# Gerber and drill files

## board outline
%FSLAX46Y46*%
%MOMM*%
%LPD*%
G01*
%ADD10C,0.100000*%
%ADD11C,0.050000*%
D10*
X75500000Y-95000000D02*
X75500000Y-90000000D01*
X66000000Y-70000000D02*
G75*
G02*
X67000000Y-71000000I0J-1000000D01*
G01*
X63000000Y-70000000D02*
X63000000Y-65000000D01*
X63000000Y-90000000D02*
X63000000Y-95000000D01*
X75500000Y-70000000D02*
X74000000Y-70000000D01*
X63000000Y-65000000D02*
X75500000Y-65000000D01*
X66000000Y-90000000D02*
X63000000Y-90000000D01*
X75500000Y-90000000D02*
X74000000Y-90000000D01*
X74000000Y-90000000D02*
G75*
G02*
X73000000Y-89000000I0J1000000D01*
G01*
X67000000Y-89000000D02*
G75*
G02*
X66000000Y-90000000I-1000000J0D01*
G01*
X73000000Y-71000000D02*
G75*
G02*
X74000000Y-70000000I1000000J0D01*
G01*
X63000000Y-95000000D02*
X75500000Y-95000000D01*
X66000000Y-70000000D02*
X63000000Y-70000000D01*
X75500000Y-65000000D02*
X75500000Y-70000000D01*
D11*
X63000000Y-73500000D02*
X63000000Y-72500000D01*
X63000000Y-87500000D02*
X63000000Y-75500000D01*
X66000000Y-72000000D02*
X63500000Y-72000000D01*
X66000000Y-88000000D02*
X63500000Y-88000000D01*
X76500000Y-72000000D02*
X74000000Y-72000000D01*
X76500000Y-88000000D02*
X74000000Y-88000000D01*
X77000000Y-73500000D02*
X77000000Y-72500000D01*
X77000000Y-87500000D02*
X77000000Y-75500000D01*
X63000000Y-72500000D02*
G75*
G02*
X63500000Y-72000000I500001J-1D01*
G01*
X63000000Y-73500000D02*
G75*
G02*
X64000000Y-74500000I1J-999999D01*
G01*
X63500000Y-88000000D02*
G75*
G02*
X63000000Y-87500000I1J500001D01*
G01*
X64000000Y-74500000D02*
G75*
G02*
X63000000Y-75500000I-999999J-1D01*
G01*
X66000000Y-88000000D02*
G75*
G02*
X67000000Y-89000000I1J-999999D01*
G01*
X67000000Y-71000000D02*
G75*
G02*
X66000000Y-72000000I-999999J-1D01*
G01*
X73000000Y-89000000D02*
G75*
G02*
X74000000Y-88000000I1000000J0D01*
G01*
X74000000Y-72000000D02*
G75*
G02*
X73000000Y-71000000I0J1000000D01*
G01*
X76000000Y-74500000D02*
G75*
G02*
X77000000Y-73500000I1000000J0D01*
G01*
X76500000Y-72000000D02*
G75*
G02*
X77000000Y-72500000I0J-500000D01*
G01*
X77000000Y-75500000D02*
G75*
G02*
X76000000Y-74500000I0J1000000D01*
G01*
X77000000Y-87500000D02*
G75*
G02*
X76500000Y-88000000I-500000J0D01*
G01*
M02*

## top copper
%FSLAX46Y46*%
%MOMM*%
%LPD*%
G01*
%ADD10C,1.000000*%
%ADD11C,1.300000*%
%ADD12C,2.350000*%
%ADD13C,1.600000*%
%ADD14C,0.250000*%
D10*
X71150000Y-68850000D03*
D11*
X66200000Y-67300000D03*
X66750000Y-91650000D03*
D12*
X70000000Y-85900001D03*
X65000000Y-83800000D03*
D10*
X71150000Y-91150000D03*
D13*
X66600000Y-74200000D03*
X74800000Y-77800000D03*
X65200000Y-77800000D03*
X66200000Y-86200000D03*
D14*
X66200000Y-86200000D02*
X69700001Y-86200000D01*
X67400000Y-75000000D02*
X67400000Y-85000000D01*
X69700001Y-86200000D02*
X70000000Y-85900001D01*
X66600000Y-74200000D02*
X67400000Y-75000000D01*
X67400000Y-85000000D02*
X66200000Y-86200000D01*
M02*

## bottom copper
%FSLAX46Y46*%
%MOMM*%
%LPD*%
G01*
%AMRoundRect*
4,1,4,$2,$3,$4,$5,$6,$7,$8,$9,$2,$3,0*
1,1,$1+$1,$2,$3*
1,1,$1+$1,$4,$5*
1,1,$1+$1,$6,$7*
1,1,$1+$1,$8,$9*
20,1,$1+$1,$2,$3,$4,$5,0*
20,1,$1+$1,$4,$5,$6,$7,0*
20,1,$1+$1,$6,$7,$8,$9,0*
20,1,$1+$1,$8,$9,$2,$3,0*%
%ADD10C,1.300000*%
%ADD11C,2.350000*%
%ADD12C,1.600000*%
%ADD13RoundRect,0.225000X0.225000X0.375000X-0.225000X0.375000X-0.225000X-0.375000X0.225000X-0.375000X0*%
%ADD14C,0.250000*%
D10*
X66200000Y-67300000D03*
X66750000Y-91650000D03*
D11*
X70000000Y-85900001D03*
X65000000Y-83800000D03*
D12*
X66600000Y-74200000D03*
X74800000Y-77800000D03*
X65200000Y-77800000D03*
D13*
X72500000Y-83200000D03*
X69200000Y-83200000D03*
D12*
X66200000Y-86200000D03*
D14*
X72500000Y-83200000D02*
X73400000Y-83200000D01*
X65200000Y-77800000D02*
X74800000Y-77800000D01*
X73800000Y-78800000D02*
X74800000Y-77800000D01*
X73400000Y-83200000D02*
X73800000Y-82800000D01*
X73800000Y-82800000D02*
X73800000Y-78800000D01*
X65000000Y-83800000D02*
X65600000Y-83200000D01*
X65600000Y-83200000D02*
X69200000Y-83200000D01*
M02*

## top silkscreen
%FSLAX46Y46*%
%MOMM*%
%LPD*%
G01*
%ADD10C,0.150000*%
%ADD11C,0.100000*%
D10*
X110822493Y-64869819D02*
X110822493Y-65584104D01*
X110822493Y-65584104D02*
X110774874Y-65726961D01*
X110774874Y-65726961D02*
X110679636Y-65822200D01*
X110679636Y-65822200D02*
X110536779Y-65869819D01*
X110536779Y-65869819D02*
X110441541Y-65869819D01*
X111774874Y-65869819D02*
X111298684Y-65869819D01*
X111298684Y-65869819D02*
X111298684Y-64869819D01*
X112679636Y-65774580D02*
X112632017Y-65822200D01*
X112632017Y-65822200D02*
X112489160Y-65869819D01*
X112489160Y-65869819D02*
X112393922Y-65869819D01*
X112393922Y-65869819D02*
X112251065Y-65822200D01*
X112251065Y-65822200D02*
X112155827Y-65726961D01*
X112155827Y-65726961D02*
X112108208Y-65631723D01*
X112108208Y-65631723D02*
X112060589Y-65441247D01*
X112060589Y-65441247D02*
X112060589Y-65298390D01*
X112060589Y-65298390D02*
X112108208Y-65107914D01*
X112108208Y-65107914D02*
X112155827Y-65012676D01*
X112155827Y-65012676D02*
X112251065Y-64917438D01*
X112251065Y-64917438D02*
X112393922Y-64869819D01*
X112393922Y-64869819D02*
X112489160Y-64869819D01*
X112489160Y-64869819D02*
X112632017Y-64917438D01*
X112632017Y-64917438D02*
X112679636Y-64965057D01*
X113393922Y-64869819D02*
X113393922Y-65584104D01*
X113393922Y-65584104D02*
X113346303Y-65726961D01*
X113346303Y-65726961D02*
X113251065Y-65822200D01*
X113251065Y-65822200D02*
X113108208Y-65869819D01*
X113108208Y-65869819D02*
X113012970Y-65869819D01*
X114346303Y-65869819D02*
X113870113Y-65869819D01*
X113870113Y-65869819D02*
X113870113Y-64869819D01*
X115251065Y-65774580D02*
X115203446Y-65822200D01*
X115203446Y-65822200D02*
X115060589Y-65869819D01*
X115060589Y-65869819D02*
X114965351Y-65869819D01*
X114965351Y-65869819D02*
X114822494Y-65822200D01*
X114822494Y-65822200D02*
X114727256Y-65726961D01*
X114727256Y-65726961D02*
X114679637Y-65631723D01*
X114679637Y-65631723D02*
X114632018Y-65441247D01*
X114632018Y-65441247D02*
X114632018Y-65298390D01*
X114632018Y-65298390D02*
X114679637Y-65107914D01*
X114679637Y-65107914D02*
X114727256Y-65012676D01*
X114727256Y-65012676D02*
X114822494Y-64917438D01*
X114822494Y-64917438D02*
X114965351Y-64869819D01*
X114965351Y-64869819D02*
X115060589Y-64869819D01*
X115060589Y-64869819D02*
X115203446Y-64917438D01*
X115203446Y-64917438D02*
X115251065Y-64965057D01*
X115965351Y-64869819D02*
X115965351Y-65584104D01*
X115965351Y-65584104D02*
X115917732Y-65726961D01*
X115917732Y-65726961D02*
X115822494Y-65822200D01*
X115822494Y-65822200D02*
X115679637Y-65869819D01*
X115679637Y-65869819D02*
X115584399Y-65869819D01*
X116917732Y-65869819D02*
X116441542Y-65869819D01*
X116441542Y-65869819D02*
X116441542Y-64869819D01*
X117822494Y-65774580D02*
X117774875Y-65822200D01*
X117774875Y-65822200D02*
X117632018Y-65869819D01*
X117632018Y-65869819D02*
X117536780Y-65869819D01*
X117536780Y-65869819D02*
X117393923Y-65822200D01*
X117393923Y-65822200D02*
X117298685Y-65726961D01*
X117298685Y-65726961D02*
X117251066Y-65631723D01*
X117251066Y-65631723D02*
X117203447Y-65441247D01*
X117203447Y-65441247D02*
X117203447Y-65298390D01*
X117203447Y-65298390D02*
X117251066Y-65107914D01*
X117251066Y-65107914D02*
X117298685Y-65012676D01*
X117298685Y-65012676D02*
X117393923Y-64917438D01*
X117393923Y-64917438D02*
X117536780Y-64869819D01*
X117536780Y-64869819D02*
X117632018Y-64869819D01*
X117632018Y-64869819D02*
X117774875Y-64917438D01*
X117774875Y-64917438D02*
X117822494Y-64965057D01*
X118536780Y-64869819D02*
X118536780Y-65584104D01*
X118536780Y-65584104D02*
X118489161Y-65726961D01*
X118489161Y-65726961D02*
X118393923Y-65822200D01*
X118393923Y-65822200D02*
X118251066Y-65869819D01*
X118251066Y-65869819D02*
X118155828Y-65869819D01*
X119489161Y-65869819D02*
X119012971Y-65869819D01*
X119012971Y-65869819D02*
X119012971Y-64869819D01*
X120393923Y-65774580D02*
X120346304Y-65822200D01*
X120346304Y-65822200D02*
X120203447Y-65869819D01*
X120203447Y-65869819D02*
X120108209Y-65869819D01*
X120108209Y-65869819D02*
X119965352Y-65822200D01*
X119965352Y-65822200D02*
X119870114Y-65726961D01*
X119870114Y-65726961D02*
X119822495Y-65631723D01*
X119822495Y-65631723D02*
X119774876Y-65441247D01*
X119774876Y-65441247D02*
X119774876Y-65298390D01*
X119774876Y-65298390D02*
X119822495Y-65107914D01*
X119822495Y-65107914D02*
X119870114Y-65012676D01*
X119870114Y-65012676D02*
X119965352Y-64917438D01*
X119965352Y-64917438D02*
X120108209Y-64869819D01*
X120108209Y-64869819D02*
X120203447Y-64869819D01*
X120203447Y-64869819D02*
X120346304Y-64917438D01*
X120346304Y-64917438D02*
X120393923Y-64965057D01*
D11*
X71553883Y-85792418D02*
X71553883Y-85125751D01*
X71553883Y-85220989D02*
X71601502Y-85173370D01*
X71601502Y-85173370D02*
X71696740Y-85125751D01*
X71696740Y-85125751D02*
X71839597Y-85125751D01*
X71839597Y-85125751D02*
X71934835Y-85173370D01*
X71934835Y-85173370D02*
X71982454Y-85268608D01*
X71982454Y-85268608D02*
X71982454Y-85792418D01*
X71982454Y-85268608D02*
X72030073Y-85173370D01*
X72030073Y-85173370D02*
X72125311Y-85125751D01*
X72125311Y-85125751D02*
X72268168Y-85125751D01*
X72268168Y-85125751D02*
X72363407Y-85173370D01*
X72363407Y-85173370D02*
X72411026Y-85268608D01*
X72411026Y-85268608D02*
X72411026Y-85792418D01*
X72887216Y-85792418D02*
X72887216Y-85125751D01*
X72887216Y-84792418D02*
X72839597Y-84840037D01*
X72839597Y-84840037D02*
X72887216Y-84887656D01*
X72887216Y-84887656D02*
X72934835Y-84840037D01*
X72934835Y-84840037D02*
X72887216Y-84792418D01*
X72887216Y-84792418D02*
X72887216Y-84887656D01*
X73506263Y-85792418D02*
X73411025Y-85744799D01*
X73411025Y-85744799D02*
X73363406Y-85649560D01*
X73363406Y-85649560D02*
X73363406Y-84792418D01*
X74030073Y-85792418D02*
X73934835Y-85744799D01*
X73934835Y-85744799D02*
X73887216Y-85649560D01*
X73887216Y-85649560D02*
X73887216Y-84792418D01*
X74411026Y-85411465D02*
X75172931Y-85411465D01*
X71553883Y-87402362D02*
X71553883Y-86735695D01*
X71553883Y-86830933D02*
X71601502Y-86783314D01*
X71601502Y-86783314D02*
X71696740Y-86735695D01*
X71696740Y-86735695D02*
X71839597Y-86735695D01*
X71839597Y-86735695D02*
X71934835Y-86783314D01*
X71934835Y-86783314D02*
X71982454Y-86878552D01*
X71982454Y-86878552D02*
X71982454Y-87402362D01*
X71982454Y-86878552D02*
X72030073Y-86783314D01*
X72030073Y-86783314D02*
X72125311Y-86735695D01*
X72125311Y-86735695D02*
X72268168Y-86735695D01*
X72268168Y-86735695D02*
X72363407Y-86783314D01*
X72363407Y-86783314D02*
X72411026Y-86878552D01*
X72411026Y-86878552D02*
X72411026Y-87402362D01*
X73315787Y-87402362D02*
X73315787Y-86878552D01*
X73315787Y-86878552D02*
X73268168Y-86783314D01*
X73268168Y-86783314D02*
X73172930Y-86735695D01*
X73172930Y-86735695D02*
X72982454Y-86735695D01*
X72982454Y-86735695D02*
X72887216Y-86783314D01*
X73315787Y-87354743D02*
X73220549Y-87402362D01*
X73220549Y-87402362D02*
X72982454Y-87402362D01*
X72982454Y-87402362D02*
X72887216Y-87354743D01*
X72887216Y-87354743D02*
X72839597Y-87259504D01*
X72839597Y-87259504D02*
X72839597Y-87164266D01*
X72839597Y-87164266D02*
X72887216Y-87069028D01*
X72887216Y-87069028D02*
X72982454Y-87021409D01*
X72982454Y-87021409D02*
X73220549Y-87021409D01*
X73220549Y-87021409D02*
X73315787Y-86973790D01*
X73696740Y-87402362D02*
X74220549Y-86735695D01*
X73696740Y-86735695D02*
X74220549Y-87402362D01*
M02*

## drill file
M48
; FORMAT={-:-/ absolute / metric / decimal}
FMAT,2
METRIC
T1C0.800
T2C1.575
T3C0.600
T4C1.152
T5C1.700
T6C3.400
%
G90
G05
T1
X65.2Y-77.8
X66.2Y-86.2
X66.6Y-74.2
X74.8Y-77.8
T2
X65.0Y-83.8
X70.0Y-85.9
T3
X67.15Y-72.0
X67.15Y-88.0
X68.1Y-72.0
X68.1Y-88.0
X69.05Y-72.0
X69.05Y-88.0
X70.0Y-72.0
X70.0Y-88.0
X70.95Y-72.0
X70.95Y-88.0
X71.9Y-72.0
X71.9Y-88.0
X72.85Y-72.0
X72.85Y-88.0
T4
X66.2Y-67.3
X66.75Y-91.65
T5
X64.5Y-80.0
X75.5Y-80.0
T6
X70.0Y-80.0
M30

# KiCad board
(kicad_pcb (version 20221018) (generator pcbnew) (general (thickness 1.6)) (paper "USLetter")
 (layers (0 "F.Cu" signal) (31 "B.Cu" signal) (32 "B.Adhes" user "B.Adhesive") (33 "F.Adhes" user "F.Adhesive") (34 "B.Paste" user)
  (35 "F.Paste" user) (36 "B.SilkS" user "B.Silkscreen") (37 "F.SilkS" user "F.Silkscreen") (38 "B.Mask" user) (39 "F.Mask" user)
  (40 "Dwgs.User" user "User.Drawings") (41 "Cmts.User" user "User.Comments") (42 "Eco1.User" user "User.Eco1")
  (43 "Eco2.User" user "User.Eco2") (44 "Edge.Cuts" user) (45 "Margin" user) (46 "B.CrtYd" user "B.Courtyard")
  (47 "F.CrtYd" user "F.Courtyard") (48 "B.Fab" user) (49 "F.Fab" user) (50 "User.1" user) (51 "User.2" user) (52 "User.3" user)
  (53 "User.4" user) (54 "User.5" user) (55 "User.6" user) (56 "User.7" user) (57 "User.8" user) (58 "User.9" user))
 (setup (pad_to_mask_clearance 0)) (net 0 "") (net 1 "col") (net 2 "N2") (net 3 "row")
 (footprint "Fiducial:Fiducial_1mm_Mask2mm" (layer "F.Cu") (at 71.15 68.85 -90)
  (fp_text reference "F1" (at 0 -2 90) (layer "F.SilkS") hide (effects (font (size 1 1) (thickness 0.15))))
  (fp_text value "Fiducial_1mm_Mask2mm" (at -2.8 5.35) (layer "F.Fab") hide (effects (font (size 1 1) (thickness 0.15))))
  (pad "" smd circle (at 0 0 270) (size 1 1) (layers "F.Cu" "F.Mask") (solder_mask_margin 0.5) (clearance 0.5)))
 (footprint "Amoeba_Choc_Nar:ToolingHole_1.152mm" (layer "F.Cu") (at 66.2 67.3 -90) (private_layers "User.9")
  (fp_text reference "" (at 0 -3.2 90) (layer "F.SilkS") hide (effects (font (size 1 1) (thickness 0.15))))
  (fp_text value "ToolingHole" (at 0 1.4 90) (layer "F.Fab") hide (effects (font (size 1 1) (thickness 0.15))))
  (pad "" np_thru_hole circle (at 0 0 270) (size 1.3 1.3) (drill 1.152) (layers "F&B.Cu" "*.Mask") (solder_mask_margin 0.074)))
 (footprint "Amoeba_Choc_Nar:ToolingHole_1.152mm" (layer "F.Cu") (at 66.75 91.65 -90) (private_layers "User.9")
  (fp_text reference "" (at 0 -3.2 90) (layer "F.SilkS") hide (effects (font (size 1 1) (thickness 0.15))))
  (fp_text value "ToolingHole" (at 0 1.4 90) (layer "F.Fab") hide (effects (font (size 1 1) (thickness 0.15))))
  (pad "" np_thru_hole circle (at 0 0 270) (size 1.3 1.3) (drill 1.152) (layers "F&B.Cu" "*.Mask") (solder_mask_margin 0.074)))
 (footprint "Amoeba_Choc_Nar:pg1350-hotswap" (layer "F.Cu") (at 70 80) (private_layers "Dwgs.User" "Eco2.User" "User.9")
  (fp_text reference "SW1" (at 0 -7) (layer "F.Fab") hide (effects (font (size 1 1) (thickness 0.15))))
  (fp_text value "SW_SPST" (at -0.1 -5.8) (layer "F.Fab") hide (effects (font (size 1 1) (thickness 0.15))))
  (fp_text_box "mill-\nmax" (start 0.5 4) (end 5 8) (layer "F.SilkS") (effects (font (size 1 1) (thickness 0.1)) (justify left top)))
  (fp_line (start -7 -6.5) (end -7 -7.5) (stroke (width 0.05) (type solid)) (layer "Edge.Cuts"))
  (fp_line (start -7 7.5) (end -7 -4.5) (stroke (width 0.05) (type solid)) (layer "Edge.Cuts"))
  (fp_line (start -4 -8) (end -6.5 -8) (stroke (width 0.05) (type solid)) (layer "Edge.Cuts"))
  (fp_line (start -4 8) (end -6.5 8) (stroke (width 0.05) (type solid)) (layer "Edge.Cuts"))
  (fp_line (start 6.5 -8) (end 4 -8) (stroke (width 0.05) (type solid)) (layer "Edge.Cuts"))
  (fp_line (start 6.5 8) (end 4 8) (stroke (width 0.05) (type solid)) (layer "Edge.Cuts"))
  (fp_line (start 7 -6.5) (end 7 -7.5) (stroke (width 0.05) (type solid)) (layer "Edge.Cuts"))
  (fp_line (start 7 7.5) (end 7 -4.5) (stroke (width 0.05) (type solid)) (layer "Edge.Cuts"))
  (fp_arc (start -7 -7.5) (mid -6.853553 -7.853553) (end -6.5 -8) (stroke (width 0.05) (type default)) (layer "Edge.Cuts"))
  (fp_arc (start -7 -6.5) (mid -6.292893 -6.207107) (end -6 -5.5) (stroke (width 0.05) (type default)) (layer "Edge.Cuts"))
  (fp_arc (start -6.5 8) (mid -6.853553 7.853553) (end -7 7.5) (stroke (width 0.05) (type default)) (layer "Edge.Cuts"))
  (fp_arc (start -6 -5.5) (mid -6.292893 -4.792893) (end -7 -4.5) (stroke (width 0.05) (type default)) (layer "Edge.Cuts"))
  (fp_arc (start -4 8) (mid -3.292893 8.292893) (end -3 9) (stroke (width 0.05) (type default)) (layer "Edge.Cuts"))
  (fp_arc (start -3 -9) (mid -3.292893 -8.292893) (end -4 -8) (stroke (width 0.05) (type default)) (layer "Edge.Cuts"))
  (fp_arc (start 3 9) (mid 3.292893 8.292893) (end 4 8) (stroke (width 0.05) (type default)) (layer "Edge.Cuts"))
  (fp_arc (start 4 -8) (mid 3.292893 -8.292893) (end 3 -9) (stroke (width 0.05) (type default)) (layer "Edge.Cuts"))
  (fp_arc (start 6 -5.5) (mid 6.292893 -6.207107) (end 7 -6.5) (stroke (width 0.05) (type default)) (layer "Edge.Cuts"))
  (fp_arc (start 6.5 -8) (mid 6.853553 -7.853553) (end 7 -7.5) (stroke (width 0.05) (type default)) (layer "Edge.Cuts"))
  (fp_arc (start 7 -4.5) (mid 6.292893 -4.792893) (end 6 -5.5) (stroke (width 0.05) (type default)) (layer "Edge.Cuts"))
  (fp_arc (start 7 7.5) (mid 6.853553 7.853553) (end 6.5 8) (stroke (width 0.05) (type default)) (layer "Edge.Cuts"))
  (pad "" np_thru_hole circle (at -5.5 0 180) (size 1.7 1.7) (drill 1.7) (layers "*.Cu" "*.Mask"))
  (pad "" np_thru_hole circle (at -2.85 -8) (size 0.6 0.6) (drill 0.6) (layers "*.Mask"))
  (pad "" np_thru_hole circle (at -2.85 8) (size 0.6 0.6) (drill 0.6) (layers "*.Mask"))
  (pad "" np_thru_hole circle (at -1.9 -8) (size 0.6 0.6) (drill 0.6) (layers "*.Mask"))
  (pad "" np_thru_hole circle (at -1.9 8) (size 0.6 0.6) (drill 0.6) (layers "*.Mask"))
  (pad "" np_thru_hole circle (at -0.95 -8) (size 0.6 0.6) (drill 0.6) (layers "*.Mask"))
  (pad "" np_thru_hole circle (at -0.95 8) (size 0.6 0.6) (drill 0.6) (layers "*.Mask"))
  (pad "" np_thru_hole circle (at 0 -8) (size 0.6 0.6) (drill 0.6) (layers "*.Mask"))
  (pad "" np_thru_hole circle (at 0 0 180) (size 3.4 3.4) (drill 3.4) (layers "*.Cu" "*.Mask"))
  (pad "" np_thru_hole circle (at 0 8) (size 0.6 0.6) (drill 0.6) (layers "*.Mask"))
  (pad "" np_thru_hole circle (at 0.95 -8) (size 0.6 0.6) (drill 0.6) (layers "*.Mask"))
  (pad "" np_thru_hole circle (at 0.95 8) (size 0.6 0.6) (drill 0.6) (layers "*.Mask"))
  (pad "" np_thru_hole circle (at 1.9 -8) (size 0.6 0.6) (drill 0.6) (layers "*.Mask"))
  (pad "" np_thru_hole circle (at 1.9 8) (size 0.6 0.6) (drill 0.6) (layers "*.Mask"))
  (pad "" np_thru_hole circle (at 2.85 -8) (size 0.6 0.6) (drill 0.6) (layers "*.Mask"))
  (pad "" np_thru_hole circle (at 2.85 8) (size 0.6 0.6) (drill 0.6) (layers "*.Mask"))
  (pad "" np_thru_hole circle (at 5.5 0 180) (size 1.7 1.7) (drill 1.7) (layers "*.Cu" "*.Mask"))
  (pad "1" thru_hole circle (at 0 5.900001 180) (size 2.35 2.35) (drill 1.5748) (layers "*.Cu" "*.Mask") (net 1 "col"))
  (pad "2" thru_hole circle (at -5 3.8 180) (size 2.35 2.35) (drill 1.5748) (layers "*.Cu" "*.Mask") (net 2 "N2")))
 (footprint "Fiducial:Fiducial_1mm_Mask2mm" (layer "F.Cu") (at 71.15 91.15 -90)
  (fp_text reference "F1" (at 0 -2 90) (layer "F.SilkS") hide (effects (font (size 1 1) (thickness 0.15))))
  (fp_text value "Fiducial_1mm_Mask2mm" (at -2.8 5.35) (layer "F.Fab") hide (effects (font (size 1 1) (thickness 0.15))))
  (pad "" smd circle (at 0 0 270) (size 1 1) (layers "F.Cu" "F.Mask") (solder_mask_margin 0.5) (clearance 0.5)))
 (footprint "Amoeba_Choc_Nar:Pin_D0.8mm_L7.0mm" (layer "B.Cu") (at 66.6 74.2 180)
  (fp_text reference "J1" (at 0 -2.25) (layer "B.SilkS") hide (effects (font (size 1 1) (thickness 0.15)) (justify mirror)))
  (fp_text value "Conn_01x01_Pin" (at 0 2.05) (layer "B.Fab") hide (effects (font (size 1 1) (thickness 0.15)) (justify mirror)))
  (pad "1" thru_hole circle (at 0 0 180) (size 1.6 1.6) (drill 0.8) (layers "*.Cu" "*.Mask") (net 1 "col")))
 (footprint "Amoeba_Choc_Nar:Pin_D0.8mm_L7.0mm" (layer "B.Cu") (at 74.8 77.8 180)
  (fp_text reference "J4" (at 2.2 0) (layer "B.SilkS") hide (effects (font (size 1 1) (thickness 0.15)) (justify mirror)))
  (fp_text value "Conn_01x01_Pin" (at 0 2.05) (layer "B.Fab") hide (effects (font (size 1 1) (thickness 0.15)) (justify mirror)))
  (pad "1" thru_hole circle (at 0 0 180) (size 1.6 1.6) (drill 0.8) (layers "*.Cu" "*.Mask") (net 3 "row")))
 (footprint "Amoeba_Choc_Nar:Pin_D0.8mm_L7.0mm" (layer "B.Cu") (at 65.2 77.8 180)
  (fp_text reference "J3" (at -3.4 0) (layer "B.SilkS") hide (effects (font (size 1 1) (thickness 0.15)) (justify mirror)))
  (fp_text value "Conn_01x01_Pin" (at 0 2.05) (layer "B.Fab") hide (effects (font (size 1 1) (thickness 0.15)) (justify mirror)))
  (pad "1" thru_hole circle (at 0 0 180) (size 1.6 1.6) (drill 0.8) (layers "*.Cu" "*.Mask") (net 3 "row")))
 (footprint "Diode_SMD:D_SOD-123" (layer "B.Cu") (at 70.85 83.2 180)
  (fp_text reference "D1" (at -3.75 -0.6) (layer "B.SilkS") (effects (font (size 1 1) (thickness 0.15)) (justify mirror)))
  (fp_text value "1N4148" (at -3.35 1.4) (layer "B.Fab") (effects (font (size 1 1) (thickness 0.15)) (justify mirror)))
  (pad "1" smd roundrect (at -1.65 0 180) (size 0.9 1.2) (layers "B.Cu" "B.Paste" "B.Mask") (roundrect_rratio 0.25) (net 3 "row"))
  (pad "2" smd roundrect (at 1.65 0 180) (size 0.9 1.2) (layers "B.Cu" "B.Paste" "B.Mask") (roundrect_rratio 0.25) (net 2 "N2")))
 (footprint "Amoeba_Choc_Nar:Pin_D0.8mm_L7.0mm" (layer "B.Cu") (at 66.2 86.2 180)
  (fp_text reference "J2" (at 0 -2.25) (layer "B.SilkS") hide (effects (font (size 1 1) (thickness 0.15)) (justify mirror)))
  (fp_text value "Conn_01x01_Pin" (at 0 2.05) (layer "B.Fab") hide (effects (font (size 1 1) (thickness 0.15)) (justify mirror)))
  (pad "1" thru_hole circle (at 0 0 180) (size 1.6 1.6) (drill 0.8) (layers "*.Cu" "*.Mask") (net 1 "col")))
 (gr_line (start 75.5 95) (end 75.5 90) (stroke (width 0.1) (type default)) (layer "Edge.Cuts"))
 (gr_arc (start 66 70) (mid 66.707107 70.292893) (end 67 71) (stroke (width 0.1) (type default)) (layer "Edge.Cuts"))
 (gr_line (start 63 70) (end 63 65) (stroke (width 0.1) (type default)) (layer "Edge.Cuts"))
 (gr_line (start 63 90) (end 63 95) (stroke (width 0.1) (type default)) (layer "Edge.Cuts"))
 (gr_line (start 75.5 70) (end 74 70) (stroke (width 0.1) (type default)) (layer "Edge.Cuts"))
 (gr_line (start 63 65) (end 75.5 65) (stroke (width 0.1) (type default)) (layer "Edge.Cuts"))
 (gr_line (start 66 90) (end 63 90) (stroke (width 0.1) (type default)) (layer "Edge.Cuts"))
 (gr_line (start 75.5 90) (end 74 90) (stroke (width 0.1) (type default)) (layer "Edge.Cuts"))
 (gr_arc (start 74 90) (mid 73.292893 89.707107) (end 73 89) (stroke (width 0.1) (type default)) (layer "Edge.Cuts"))
 (gr_arc (start 67 89) (mid 66.707107 89.707107) (end 66 90) (stroke (width 0.1) (type default)) (layer "Edge.Cuts"))
 (gr_arc (start 73 71) (mid 73.292893 70.292893) (end 74 70) (stroke (width 0.1) (type default)) (layer "Edge.Cuts"))
 (gr_line (start 63 95) (end 75.5 95) (stroke (width 0.1) (type default)) (layer "Edge.Cuts"))
 (gr_line (start 66 70) (end 63 70) (stroke (width 0.1) (type default)) (layer "Edge.Cuts"))
 (gr_line (start 75.5 65) (end 75.5 70) (stroke (width 0.1) (type default)) (layer "Edge.Cuts"))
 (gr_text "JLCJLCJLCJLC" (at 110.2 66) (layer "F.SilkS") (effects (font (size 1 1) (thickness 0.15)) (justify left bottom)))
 (segment (start 72.5 83.2) (end 73.4 83.2) (width 0.25) (layer "B.Cu") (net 3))
 (segment (start 65.2 77.8) (end 74.8 77.8) (width 0.25) (layer "B.Cu") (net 3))
 (segment (start 73.8 78.8) (end 74.8 77.8) (width 0.25) (layer "B.Cu") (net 3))
 (segment (start 73.4 83.2) (end 73.8 82.8) (width 0.25) (layer "B.Cu") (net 3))
 (segment (start 73.8 82.8) (end 73.8 78.8) (width 0.25) (layer "B.Cu") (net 3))
 (segment (start 65 83.8) (end 65.6 83.2) (width 0.25) (layer "B.Cu") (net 2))
 (segment (start 65.6 83.2) (end 69.2 83.2) (width 0.25) (layer "B.Cu") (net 2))
 (segment (start 66.2 86.2) (end 69.700001 86.2) (width 0.25) (layer "F.Cu") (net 1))
 (segment (start 67.4 75) (end 67.4 85) (width 0.25) (layer "F.Cu") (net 1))
 (segment (start 69.700001 86.2) (end 70 85.900001) (width 0.25) (layer "F.Cu") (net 1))
 (segment (start 66.6 74.2) (end 67.4 75) (width 0.25) (layer "F.Cu") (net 1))
 (segment (start 67.4 85) (end 66.2 86.2) (width 0.25) (layer "F.Cu") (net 1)))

